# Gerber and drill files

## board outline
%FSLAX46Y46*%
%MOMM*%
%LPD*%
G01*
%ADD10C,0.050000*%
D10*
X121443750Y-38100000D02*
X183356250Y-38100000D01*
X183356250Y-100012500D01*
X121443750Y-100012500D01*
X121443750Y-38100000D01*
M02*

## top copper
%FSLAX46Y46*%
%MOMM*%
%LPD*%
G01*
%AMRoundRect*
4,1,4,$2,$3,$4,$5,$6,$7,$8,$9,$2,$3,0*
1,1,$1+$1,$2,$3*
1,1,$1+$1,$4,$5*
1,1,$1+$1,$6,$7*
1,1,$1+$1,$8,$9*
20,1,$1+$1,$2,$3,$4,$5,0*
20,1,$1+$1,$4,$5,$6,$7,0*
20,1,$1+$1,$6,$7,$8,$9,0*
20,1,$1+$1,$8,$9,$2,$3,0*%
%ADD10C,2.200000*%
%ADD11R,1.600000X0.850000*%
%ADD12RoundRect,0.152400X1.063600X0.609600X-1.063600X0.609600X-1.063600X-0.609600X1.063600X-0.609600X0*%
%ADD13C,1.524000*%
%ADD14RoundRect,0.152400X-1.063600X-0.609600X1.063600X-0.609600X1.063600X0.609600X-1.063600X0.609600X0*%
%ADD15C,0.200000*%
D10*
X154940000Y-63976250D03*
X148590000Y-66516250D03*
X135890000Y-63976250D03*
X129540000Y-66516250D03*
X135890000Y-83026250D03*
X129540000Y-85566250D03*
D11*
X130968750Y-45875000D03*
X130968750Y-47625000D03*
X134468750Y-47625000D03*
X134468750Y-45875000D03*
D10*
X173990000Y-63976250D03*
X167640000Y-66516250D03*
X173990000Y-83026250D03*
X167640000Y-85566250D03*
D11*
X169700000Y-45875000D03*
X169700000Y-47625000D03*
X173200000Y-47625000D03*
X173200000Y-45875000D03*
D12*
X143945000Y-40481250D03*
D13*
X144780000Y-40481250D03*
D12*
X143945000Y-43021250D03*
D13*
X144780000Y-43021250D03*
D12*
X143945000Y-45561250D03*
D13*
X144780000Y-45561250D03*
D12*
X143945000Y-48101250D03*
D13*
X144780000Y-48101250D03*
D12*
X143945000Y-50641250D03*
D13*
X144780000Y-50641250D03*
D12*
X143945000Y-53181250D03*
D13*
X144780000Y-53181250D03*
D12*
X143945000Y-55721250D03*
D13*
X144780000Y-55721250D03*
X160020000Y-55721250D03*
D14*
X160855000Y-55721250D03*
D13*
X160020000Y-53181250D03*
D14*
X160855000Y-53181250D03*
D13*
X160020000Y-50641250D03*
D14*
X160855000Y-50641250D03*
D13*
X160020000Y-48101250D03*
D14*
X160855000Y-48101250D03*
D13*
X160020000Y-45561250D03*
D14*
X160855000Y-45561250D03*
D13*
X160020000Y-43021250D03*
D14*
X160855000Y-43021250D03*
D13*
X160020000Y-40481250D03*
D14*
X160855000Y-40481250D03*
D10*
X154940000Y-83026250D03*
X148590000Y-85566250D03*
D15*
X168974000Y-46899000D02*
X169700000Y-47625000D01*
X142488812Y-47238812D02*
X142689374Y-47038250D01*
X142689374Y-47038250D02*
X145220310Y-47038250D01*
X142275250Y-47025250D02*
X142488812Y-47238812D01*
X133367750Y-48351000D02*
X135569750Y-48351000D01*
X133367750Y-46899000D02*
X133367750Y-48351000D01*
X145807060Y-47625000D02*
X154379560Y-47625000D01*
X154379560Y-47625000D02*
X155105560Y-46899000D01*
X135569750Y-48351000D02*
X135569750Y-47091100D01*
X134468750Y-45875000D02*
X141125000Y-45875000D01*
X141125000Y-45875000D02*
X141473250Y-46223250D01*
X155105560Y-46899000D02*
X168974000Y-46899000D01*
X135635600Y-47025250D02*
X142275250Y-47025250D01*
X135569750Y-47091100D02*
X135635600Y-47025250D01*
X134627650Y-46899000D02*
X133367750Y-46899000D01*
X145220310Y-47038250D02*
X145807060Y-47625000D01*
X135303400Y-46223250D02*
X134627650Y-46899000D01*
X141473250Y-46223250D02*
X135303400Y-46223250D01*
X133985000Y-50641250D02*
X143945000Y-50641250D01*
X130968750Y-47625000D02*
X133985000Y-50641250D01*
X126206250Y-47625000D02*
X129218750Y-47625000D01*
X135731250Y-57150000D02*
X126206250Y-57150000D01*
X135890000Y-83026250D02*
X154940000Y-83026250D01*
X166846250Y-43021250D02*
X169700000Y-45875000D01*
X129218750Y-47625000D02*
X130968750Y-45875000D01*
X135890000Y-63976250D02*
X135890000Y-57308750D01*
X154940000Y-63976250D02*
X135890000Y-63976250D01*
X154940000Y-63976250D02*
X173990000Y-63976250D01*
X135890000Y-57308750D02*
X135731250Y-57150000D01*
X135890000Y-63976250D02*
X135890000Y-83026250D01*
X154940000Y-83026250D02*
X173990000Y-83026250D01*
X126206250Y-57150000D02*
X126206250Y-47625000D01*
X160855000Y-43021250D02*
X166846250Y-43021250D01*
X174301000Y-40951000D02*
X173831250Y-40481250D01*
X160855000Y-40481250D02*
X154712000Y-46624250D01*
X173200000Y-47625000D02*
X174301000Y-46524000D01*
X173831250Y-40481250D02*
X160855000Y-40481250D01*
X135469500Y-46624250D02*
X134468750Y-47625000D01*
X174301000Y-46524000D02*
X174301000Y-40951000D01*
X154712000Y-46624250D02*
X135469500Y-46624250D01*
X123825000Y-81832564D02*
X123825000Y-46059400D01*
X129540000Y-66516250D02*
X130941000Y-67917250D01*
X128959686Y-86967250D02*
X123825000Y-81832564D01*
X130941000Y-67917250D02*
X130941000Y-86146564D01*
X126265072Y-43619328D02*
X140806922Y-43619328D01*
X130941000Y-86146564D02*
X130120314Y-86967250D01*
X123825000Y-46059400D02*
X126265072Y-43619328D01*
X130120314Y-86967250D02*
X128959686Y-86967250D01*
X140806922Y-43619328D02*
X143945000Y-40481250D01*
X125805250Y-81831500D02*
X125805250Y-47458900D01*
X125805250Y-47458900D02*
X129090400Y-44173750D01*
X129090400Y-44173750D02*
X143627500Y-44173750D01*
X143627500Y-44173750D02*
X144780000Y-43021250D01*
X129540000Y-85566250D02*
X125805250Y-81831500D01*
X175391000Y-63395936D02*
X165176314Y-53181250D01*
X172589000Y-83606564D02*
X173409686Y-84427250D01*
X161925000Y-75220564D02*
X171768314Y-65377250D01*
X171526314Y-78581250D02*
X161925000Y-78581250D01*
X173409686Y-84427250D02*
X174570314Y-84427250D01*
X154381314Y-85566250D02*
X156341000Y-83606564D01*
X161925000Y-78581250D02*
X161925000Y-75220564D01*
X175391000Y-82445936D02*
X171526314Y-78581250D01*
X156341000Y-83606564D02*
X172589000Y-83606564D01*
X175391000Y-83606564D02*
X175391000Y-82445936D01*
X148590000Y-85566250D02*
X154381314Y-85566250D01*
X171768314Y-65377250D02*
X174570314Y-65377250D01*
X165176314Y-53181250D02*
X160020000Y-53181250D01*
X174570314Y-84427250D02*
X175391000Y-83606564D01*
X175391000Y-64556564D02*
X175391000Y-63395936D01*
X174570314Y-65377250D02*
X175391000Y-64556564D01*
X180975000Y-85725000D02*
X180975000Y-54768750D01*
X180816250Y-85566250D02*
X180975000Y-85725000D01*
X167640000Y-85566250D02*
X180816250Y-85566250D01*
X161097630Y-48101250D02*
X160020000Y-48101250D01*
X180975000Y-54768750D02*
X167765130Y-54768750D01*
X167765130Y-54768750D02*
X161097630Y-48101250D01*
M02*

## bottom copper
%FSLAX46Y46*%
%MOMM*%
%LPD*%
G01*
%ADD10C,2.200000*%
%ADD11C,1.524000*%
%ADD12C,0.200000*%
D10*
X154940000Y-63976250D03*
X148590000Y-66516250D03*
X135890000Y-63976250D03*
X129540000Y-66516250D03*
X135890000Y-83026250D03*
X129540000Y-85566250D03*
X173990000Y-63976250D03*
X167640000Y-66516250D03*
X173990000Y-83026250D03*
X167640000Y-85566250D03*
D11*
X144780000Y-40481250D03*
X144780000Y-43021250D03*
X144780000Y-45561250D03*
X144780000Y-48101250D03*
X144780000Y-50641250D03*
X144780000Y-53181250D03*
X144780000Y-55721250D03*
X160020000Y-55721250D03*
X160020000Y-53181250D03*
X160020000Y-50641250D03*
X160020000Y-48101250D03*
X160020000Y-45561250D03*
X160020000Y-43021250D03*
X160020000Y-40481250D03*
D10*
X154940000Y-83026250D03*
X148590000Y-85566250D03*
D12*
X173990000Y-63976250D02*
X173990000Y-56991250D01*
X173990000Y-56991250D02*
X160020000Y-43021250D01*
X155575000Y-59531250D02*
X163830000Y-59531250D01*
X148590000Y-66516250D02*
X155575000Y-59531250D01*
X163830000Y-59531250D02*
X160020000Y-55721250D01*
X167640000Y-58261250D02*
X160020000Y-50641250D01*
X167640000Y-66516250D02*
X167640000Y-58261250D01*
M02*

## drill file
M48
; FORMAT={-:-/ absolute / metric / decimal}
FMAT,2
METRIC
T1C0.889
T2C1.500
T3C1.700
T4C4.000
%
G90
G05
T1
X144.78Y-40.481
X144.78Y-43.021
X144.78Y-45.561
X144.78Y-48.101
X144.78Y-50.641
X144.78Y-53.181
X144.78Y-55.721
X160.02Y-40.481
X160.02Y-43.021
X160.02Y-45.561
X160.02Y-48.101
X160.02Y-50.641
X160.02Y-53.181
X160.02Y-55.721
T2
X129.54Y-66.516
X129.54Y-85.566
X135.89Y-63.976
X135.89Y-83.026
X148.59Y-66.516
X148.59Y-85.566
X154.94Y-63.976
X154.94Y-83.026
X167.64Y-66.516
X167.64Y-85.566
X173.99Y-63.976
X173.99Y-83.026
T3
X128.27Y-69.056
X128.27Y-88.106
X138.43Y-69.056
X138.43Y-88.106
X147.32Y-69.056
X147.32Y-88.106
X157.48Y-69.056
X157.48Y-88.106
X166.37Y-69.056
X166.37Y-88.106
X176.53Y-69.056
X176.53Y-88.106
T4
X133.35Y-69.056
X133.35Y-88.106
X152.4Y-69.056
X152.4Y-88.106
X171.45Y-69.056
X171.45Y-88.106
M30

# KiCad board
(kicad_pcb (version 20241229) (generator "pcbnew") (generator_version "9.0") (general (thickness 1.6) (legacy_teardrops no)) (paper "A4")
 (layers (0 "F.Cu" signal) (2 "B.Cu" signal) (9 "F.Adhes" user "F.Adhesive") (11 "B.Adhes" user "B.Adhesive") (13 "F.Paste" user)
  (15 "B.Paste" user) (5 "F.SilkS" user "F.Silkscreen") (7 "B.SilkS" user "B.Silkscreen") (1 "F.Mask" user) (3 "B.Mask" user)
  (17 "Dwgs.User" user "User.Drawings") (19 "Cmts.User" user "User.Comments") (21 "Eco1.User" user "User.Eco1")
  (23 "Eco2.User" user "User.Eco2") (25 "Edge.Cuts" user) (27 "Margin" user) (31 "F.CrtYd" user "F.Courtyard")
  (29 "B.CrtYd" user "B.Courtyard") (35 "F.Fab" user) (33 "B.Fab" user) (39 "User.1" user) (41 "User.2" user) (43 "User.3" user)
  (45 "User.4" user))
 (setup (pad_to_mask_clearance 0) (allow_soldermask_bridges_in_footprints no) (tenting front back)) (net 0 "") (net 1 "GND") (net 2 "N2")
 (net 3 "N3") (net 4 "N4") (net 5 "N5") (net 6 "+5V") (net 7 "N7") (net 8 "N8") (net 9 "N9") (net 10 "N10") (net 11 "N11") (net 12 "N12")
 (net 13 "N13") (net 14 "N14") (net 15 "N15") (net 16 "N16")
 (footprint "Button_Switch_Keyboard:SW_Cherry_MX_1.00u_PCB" (layer "F.Cu") (at 154.94 63.97625)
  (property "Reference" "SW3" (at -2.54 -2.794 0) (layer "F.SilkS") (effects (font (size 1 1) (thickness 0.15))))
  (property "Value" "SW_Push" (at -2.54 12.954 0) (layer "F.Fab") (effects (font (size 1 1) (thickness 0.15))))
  (pad "" np_thru_hole circle (at -7.62 5.08) (size 1.7 1.7) (drill 1.7) (layers "*.Cu" "*.Mask"))
  (pad "" np_thru_hole circle (at -2.54 5.08) (size 4 4) (drill 4) (layers "*.Cu" "*.Mask"))
  (pad "" np_thru_hole circle (at 2.54 5.08) (size 1.7 1.7) (drill 1.7) (layers "*.Cu" "*.Mask"))
  (pad "1" thru_hole circle (at 0 0) (size 2.2 2.2) (drill 1.5) (layers "*.Cu" "*.Mask") (remove_unused_layers no) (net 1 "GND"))
  (pad "2" thru_hole circle (at -6.35 2.54) (size 2.2 2.2) (drill 1.5) (layers "*.Cu" "*.Mask") (remove_unused_layers no) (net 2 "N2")))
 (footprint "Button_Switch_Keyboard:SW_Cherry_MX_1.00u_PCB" (layer "F.Cu") (at 135.89 63.97625)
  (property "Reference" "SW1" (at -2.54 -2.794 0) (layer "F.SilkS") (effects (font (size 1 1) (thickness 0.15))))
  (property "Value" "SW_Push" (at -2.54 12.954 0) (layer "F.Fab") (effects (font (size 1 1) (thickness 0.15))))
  (pad "" np_thru_hole circle (at -7.62 5.08) (size 1.7 1.7) (drill 1.7) (layers "*.Cu" "*.Mask"))
  (pad "" np_thru_hole circle (at -2.54 5.08) (size 4 4) (drill 4) (layers "*.Cu" "*.Mask"))
  (pad "" np_thru_hole circle (at 2.54 5.08) (size 1.7 1.7) (drill 1.7) (layers "*.Cu" "*.Mask"))
  (pad "1" thru_hole circle (at 0 0) (size 2.2 2.2) (drill 1.5) (layers "*.Cu" "*.Mask") (remove_unused_layers no) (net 1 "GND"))
  (pad "2" thru_hole circle (at -6.35 2.54) (size 2.2 2.2) (drill 1.5) (layers "*.Cu" "*.Mask") (remove_unused_layers no) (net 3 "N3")))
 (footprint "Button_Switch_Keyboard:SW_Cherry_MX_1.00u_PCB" (layer "F.Cu") (at 135.89 83.02625)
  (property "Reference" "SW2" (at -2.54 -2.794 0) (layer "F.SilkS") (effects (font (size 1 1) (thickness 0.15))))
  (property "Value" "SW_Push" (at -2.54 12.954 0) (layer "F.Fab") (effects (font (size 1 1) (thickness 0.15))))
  (pad "" np_thru_hole circle (at -7.62 5.08) (size 1.7 1.7) (drill 1.7) (layers "*.Cu" "*.Mask"))
  (pad "" np_thru_hole circle (at -2.54 5.08) (size 4 4) (drill 4) (layers "*.Cu" "*.Mask"))
  (pad "" np_thru_hole circle (at 2.54 5.08) (size 1.7 1.7) (drill 1.7) (layers "*.Cu" "*.Mask"))
  (pad "1" thru_hole circle (at 0 0) (size 2.2 2.2) (drill 1.5) (layers "*.Cu" "*.Mask") (remove_unused_layers no) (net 1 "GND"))
  (pad "2" thru_hole circle (at -6.35 2.54) (size 2.2 2.2) (drill 1.5) (layers "*.Cu" "*.Mask") (remove_unused_layers no) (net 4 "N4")))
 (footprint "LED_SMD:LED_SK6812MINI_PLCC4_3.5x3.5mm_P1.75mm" (layer "F.Cu") (at 132.71875 46.75)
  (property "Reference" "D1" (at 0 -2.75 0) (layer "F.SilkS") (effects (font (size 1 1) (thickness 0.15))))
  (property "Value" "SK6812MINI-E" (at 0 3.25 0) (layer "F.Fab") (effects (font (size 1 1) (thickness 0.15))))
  (pad "1" smd rect (at -1.75 -0.875) (size 1.6 0.85) (layers "F.Cu" "F.Mask" "F.Paste") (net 1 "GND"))
  (pad "2" smd rect (at -1.75 0.875) (size 1.6 0.85) (layers "F.Cu" "F.Mask" "F.Paste") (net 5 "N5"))
  (pad "3" smd rect (at 1.75 0.875) (size 1.6 0.85) (layers "F.Cu" "F.Mask" "F.Paste") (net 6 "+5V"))
  (pad "4" smd rect (at 1.75 -0.875) (size 1.6 0.85) (layers "F.Cu" "F.Mask" "F.Paste") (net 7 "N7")))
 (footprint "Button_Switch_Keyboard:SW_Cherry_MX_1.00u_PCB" (layer "F.Cu") (at 173.99 63.97625)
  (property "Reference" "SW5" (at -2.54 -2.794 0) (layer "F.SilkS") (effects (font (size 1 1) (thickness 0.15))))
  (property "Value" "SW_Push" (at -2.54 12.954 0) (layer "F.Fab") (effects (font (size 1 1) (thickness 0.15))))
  (pad "" np_thru_hole circle (at -7.62 5.08) (size 1.7 1.7) (drill 1.7) (layers "*.Cu" "*.Mask"))
  (pad "" np_thru_hole circle (at -2.54 5.08) (size 4 4) (drill 4) (layers "*.Cu" "*.Mask"))
  (pad "" np_thru_hole circle (at 2.54 5.08) (size 1.7 1.7) (drill 1.7) (layers "*.Cu" "*.Mask"))
  (pad "1" thru_hole circle (at 0 0) (size 2.2 2.2) (drill 1.5) (layers "*.Cu" "*.Mask") (remove_unused_layers no) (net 1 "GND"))
  (pad "2" thru_hole circle (at -6.35 2.54) (size 2.2 2.2) (drill 1.5) (layers "*.Cu" "*.Mask") (remove_unused_layers no) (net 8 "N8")))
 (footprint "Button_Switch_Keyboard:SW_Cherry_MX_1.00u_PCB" (layer "F.Cu") (at 173.99 83.02625)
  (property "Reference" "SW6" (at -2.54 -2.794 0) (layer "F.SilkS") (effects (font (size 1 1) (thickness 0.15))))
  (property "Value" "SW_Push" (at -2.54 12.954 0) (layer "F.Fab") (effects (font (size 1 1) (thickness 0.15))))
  (pad "" np_thru_hole circle (at -7.62 5.08) (size 1.7 1.7) (drill 1.7) (layers "*.Cu" "*.Mask"))
  (pad "" np_thru_hole circle (at -2.54 5.08) (size 4 4) (drill 4) (layers "*.Cu" "*.Mask"))
  (pad "" np_thru_hole circle (at 2.54 5.08) (size 1.7 1.7) (drill 1.7) (layers "*.Cu" "*.Mask"))
  (pad "1" thru_hole circle (at 0 0) (size 2.2 2.2) (drill 1.5) (layers "*.Cu" "*.Mask") (remove_unused_layers no) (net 1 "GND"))
  (pad "2" thru_hole circle (at -6.35 2.54) (size 2.2 2.2) (drill 1.5) (layers "*.Cu" "*.Mask") (remove_unused_layers no) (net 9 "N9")))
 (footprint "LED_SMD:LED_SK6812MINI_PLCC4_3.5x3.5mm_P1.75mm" (layer "F.Cu") (at 171.45 46.75)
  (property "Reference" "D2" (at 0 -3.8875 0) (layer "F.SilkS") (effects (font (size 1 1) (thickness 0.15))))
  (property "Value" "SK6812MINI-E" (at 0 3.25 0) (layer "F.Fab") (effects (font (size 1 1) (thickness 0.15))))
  (pad "1" smd rect (at -1.75 -0.875) (size 1.6 0.85) (layers "F.Cu" "F.Mask" "F.Paste") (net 1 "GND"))
  (pad "2" smd rect (at -1.75 0.875) (size 1.6 0.85) (layers "F.Cu" "F.Mask" "F.Paste") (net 7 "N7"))
  (pad "3" smd rect (at 1.75 0.875) (size 1.6 0.85) (layers "F.Cu" "F.Mask" "F.Paste") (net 6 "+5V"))
  (pad "4" smd rect (at 1.75 -0.875) (size 1.6 0.85) (layers "F.Cu" "F.Mask" "F.Paste") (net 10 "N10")))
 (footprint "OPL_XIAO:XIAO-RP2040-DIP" (layer "F.Cu") (at 152.4 48.10125)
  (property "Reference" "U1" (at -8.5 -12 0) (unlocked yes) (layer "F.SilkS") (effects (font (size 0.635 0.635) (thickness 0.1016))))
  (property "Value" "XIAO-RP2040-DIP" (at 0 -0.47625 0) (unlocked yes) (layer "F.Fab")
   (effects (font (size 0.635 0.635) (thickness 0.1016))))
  (pad "1" smd roundrect (at -8.455 -7.62 180) (size 2.432 1.524) (layers "F.Cu" "F.Mask") (roundrect_rratio 0.1) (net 3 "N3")
   (thermal_bridge_angle 45))
  (pad "1" thru_hole circle (at -7.62 -7.62 180) (size 1.524 1.524) (drill 0.889) (layers "*.Cu" "*.Mask") (remove_unused_layers no)
   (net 3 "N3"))
  (pad "2" smd roundrect (at -8.455 -5.08 180) (size 2.432 1.524) (layers "F.Cu" "F.Mask") (roundrect_rratio 0.1) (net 4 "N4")
   (thermal_bridge_angle 45))
  (pad "2" thru_hole circle (at -7.62 -5.08 180) (size 1.524 1.524) (drill 0.889) (layers "*.Cu" "*.Mask") (remove_unused_layers no)
   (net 4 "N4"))
  (pad "3" smd roundrect (at -8.455 -2.54 180) (size 2.432 1.524) (layers "F.Cu" "F.Mask") (roundrect_rratio 0.1) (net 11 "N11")
   (thermal_bridge_angle 45))
  (pad "3" thru_hole circle (at -7.62 -2.54 180) (size 1.524 1.524) (drill 0.889) (layers "*.Cu" "*.Mask") (remove_unused_layers no)
   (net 11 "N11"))
  (pad "4" smd roundrect (at -8.455 0 180) (size 2.432 1.524) (layers "F.Cu" "F.Mask") (roundrect_rratio 0.1) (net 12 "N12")
   (thermal_bridge_angle 45))
  (pad "4" thru_hole circle (at -7.62 0 180) (size 1.524 1.524) (drill 0.889) (layers "*.Cu" "*.Mask") (remove_unused_layers no)
   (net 12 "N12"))
  (pad "5" smd roundrect (at -8.455 2.54 180) (size 2.432 1.524) (layers "F.Cu" "F.Mask") (roundrect_rratio 0.1) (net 5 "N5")
   (thermal_bridge_angle 45))
  (pad "5" thru_hole circle (at -7.62 2.54 180) (size 1.524 1.524) (drill 0.889) (layers "*.Cu" "*.Mask") (remove_unused_layers no)
   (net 5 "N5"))
  (pad "6" smd roundrect (at -8.455 5.08 180) (size 2.432 1.524) (layers "F.Cu" "F.Mask") (roundrect_rratio 0.1) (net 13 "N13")
   (thermal_bridge_angle 45))
  (pad "6" thru_hole circle (at -7.62 5.08 180) (size 1.524 1.524) (drill 0.889) (layers "*.Cu" "*.Mask") (remove_unused_layers no)
   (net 13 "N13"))
  (pad "7" smd roundrect (at -8.455 7.62 180) (size 2.432 1.524) (layers "F.Cu" "F.Mask") (roundrect_rratio 0.1) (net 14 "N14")
   (thermal_bridge_angle 45))
  (pad "7" thru_hole circle (at -7.62 7.62 180) (size 1.524 1.524) (drill 0.889) (layers "*.Cu" "*.Mask") (remove_unused_layers no)
   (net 14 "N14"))
  (pad "8" thru_hole circle (at 7.62 7.62) (size 1.524 1.524) (drill 0.889) (layers "*.Cu" "*.Mask") (remove_unused_layers no) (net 2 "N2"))
  (pad "8" smd roundrect (at 8.455 7.62) (size 2.432 1.524) (layers "F.Cu" "F.Mask") (roundrect_rratio 0.1) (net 2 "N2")
   (thermal_bridge_angle 45))
  (pad "9" thru_hole circle (at 7.62 5.08) (size 1.524 1.524) (drill 0.889) (layers "*.Cu" "*.Mask") (remove_unused_layers no)
   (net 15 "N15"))
  (pad "9" smd roundrect (at 8.455 5.08) (size 2.432 1.524) (layers "F.Cu" "F.Mask") (roundrect_rratio 0.1) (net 15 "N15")
   (thermal_bridge_angle 45))
  (pad "10" thru_hole circle (at 7.62 2.54) (size 1.524 1.524) (drill 0.889) (layers "*.Cu" "*.Mask") (remove_unused_layers no) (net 8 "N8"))
  (pad "10" smd roundrect (at 8.455 2.54) (size 2.432 1.524) (layers "F.Cu" "F.Mask") (roundrect_rratio 0.1) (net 8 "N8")
   (thermal_bridge_angle 45))
  (pad "11" thru_hole circle (at 7.62 0) (size 1.524 1.524) (drill 0.889) (layers "*.Cu" "*.Mask") (remove_unused_layers no) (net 9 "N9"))
  (pad "11" smd roundrect (at 8.455 0) (size 2.432 1.524) (layers "F.Cu" "F.Mask") (roundrect_rratio 0.1) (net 9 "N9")
   (thermal_bridge_angle 45))
  (pad "12" thru_hole circle (at 7.62 -2.54) (size 1.524 1.524) (drill 0.889) (layers "*.Cu" "*.Mask") (remove_unused_layers no)
   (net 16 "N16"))
  (pad "12" smd roundrect (at 8.455 -2.54) (size 2.432 1.524) (layers "F.Cu" "F.Mask") (roundrect_rratio 0.1) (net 16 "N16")
   (thermal_bridge_angle 45))
  (pad "13" thru_hole circle (at 7.62 -5.08) (size 1.524 1.524) (drill 0.889) (layers "*.Cu" "*.Mask") (remove_unused_layers no)
   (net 1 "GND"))
  (pad "13" smd roundrect (at 8.455 -5.08) (size 2.432 1.524) (layers "F.Cu" "F.Mask") (roundrect_rratio 0.1) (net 1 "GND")
   (thermal_bridge_angle 45))
  (pad "14" thru_hole circle (at 7.62 -7.62) (size 1.524 1.524) (drill 0.889) (layers "*.Cu" "*.Mask") (remove_unused_layers no)
   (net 6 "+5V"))
  (pad "14" smd roundrect (at 8.455 -7.62) (size 2.432 1.524) (layers "F.Cu" "F.Mask") (roundrect_rratio 0.1) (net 6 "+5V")
   (thermal_bridge_angle 45)))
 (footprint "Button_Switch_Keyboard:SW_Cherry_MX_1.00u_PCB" (layer "F.Cu") (at 154.94 83.02625)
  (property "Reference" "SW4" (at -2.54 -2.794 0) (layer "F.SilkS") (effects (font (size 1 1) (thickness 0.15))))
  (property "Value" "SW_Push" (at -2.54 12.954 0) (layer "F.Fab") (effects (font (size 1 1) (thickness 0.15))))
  (pad "" np_thru_hole circle (at -7.62 5.08) (size 1.7 1.7) (drill 1.7) (layers "*.Cu" "*.Mask"))
  (pad "" np_thru_hole circle (at -2.54 5.08) (size 4 4) (drill 4) (layers "*.Cu" "*.Mask"))
  (pad "" np_thru_hole circle (at 2.54 5.08) (size 1.7 1.7) (drill 1.7) (layers "*.Cu" "*.Mask"))
  (pad "1" thru_hole circle (at 0 0) (size 2.2 2.2) (drill 1.5) (layers "*.Cu" "*.Mask") (remove_unused_layers no) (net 1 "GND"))
  (pad "2" thru_hole circle (at -6.35 2.54) (size 2.2 2.2) (drill 1.5) (layers "*.Cu" "*.Mask") (remove_unused_layers no) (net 15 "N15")))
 (gr_rect (start 121.44375 38.1) (end 183.35625 100.0125) (stroke (width 0.05) (type default)) (fill no) (layer "Edge.Cuts"))
 (segment (start 168.974 46.899) (end 169.7 47.625) (width 0.2) (layer "F.Cu") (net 7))
 (segment (start 142.488812 47.238812) (end 142.689374 47.03825) (width 0.2) (layer "F.Cu") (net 7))
 (segment (start 142.689374 47.03825) (end 145.22031 47.03825) (width 0.2) (layer "F.Cu") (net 7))
 (segment (start 142.27525 47.02525) (end 142.488812 47.238812) (width 0.2) (layer "F.Cu") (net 7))
 (segment (start 133.36775 48.351) (end 135.56975 48.351) (width 0.2) (layer "F.Cu") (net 7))
 (segment (start 133.36775 46.899) (end 133.36775 48.351) (width 0.2) (layer "F.Cu") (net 7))
 (segment (start 145.80706 47.625) (end 154.37956 47.625) (width 0.2) (layer "F.Cu") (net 7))
 (segment (start 154.37956 47.625) (end 155.10556 46.899) (width 0.2) (layer "F.Cu") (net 7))
 (segment (start 135.56975 48.351) (end 135.56975 47.0911) (width 0.2) (layer "F.Cu") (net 7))
 (segment (start 134.46875 45.875) (end 141.125 45.875) (width 0.2) (layer "F.Cu") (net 7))
 (segment (start 141.125 45.875) (end 141.47325 46.22325) (width 0.2) (layer "F.Cu") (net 7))
 (segment (start 155.10556 46.899) (end 168.974 46.899) (width 0.2) (layer "F.Cu") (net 7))
 (segment (start 135.6356 47.02525) (end 142.27525 47.02525) (width 0.2) (layer "F.Cu") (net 7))
 (segment (start 135.56975 47.0911) (end 135.6356 47.02525) (width 0.2) (layer "F.Cu") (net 7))
 (segment (start 134.62765 46.899) (end 133.36775 46.899) (width 0.2) (layer "F.Cu") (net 7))
 (segment (start 145.22031 47.03825) (end 145.80706 47.625) (width 0.2) (layer "F.Cu") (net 7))
 (segment (start 135.3034 46.22325) (end 134.62765 46.899) (width 0.2) (layer "F.Cu") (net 7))
 (segment (start 141.47325 46.22325) (end 135.3034 46.22325) (width 0.2) (layer "F.Cu") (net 7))
 (segment (start 133.985 50.64125) (end 143.945 50.64125) (width 0.2) (layer "F.Cu") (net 5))
 (segment (start 130.96875 47.625) (end 133.985 50.64125) (width 0.2) (layer "F.Cu") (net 5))
 (segment (start 126.20625 47.625) (end 129.21875 47.625) (width 0.2) (layer "F.Cu") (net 1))
 (segment (start 135.73125 57.15) (end 126.20625 57.15) (width 0.2) (layer "F.Cu") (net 1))
 (segment (start 135.89 83.02625) (end 154.94 83.02625) (width 0.2) (layer "F.Cu") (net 1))
 (segment (start 166.84625 43.02125) (end 169.7 45.875) (width 0.2) (layer "F.Cu") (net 1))
 (segment (start 129.21875 47.625) (end 130.96875 45.875) (width 0.2) (layer "F.Cu") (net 1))
 (segment (start 135.89 63.97625) (end 135.89 57.30875) (width 0.2) (layer "F.Cu") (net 1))
 (segment (start 154.94 63.97625) (end 135.89 63.97625) (width 0.2) (layer "F.Cu") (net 1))
 (segment (start 154.94 63.97625) (end 173.99 63.97625) (width 0.2) (layer "F.Cu") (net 1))
 (segment (start 135.89 57.30875) (end 135.73125 57.15) (width 0.2) (layer "F.Cu") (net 1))
 (segment (start 135.89 63.97625) (end 135.89 83.02625) (width 0.2) (layer "F.Cu") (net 1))
 (segment (start 154.94 83.02625) (end 173.99 83.02625) (width 0.2) (layer "F.Cu") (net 1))
 (segment (start 126.20625 57.15) (end 126.20625 47.625) (width 0.2) (layer "F.Cu") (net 1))
 (segment (start 160.855 43.02125) (end 166.84625 43.02125) (width 0.2) (layer "F.Cu") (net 1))
 (segment (start 173.99 63.97625) (end 173.99 56.99125) (width 0.2) (layer "B.Cu") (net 1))
 (segment (start 173.99 56.99125) (end 160.02 43.02125) (width 0.2) (layer "B.Cu") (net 1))
 (segment (start 174.301 40.951) (end 173.83125 40.48125) (width 0.2) (layer "F.Cu") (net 6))
 (segment (start 160.855 40.48125) (end 154.712 46.62425) (width 0.2) (layer "F.Cu") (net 6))
 (segment (start 173.2 47.625) (end 174.301 46.524) (width 0.2) (layer "F.Cu") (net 6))
 (segment (start 173.83125 40.48125) (end 160.855 40.48125) (width 0.2) (layer "F.Cu") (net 6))
 (segment (start 135.4695 46.62425) (end 134.46875 47.625) (width 0.2) (layer "F.Cu") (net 6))
 (segment (start 174.301 46.524) (end 174.301 40.951) (width 0.2) (layer "F.Cu") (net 6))
 (segment (start 154.712 46.62425) (end 135.4695 46.62425) (width 0.2) (layer "F.Cu") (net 6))
 (segment (start 123.825 81.832564) (end 123.825 46.0594) (width 0.2) (layer "F.Cu") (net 3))
 (segment (start 129.54 66.51625) (end 130.941 67.91725) (width 0.2) (layer "F.Cu") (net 3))
 (segment (start 128.959686 86.96725) (end 123.825 81.832564) (width 0.2) (layer "F.Cu") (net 3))
 (segment (start 130.941 67.91725) (end 130.941 86.146564) (width 0.2) (layer "F.Cu") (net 3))
 (segment (start 126.265072 43.619328) (end 140.806922 43.619328) (width 0.2) (layer "F.Cu") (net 3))
 (segment (start 130.941 86.146564) (end 130.120314 86.96725) (width 0.2) (layer "F.Cu") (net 3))
 (segment (start 123.825 46.0594) (end 126.265072 43.619328) (width 0.2) (layer "F.Cu") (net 3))
 (segment (start 130.120314 86.96725) (end 128.959686 86.96725) (width 0.2) (layer "F.Cu") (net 3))
 (segment (start 140.806922 43.619328) (end 143.945 40.48125) (width 0.2) (layer "F.Cu") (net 3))
 (segment (start 125.80525 81.8315) (end 125.80525 47.4589) (width 0.2) (layer "F.Cu") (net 4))
 (segment (start 125.80525 47.4589) (end 129.0904 44.17375) (width 0.2) (layer "F.Cu") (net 4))
 (segment (start 129.0904 44.17375) (end 143.6275 44.17375) (width 0.2) (layer "F.Cu") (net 4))
 (segment (start 143.6275 44.17375) (end 144.78 43.02125) (width 0.2) (layer "F.Cu") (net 4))
 (segment (start 129.54 85.56625) (end 125.80525 81.8315) (width 0.2) (layer "F.Cu") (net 4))
 (segment (start 155.575 59.53125) (end 163.83 59.53125) (width 0.2) (layer "B.Cu") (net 2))
 (segment (start 148.59 66.51625) (end 155.575 59.53125) (width 0.2) (layer "B.Cu") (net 2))
 (segment (start 163.83 59.53125) (end 160.02 55.72125) (width 0.2) (layer "B.Cu") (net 2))
 (segment (start 175.391 63.395936) (end 165.176314 53.18125) (width 0.2) (layer "F.Cu") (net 15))
 (segment (start 172.589 83.606564) (end 173.409686 84.42725) (width 0.2) (layer "F.Cu") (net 15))
 (segment (start 161.925 75.220564) (end 171.768314 65.37725) (width 0.2) (layer "F.Cu") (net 15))
 (segment (start 171.526314 78.58125) (end 161.925 78.58125) (width 0.2) (layer "F.Cu") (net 15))
 (segment (start 173.409686 84.42725) (end 174.570314 84.42725) (width 0.2) (layer "F.Cu") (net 15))
 (segment (start 154.381314 85.56625) (end 156.341 83.606564) (width 0.2) (layer "F.Cu") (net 15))
 (segment (start 161.925 78.58125) (end 161.925 75.220564) (width 0.2) (layer "F.Cu") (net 15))
 (segment (start 175.391 82.445936) (end 171.526314 78.58125) (width 0.2) (layer "F.Cu") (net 15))
 (segment (start 156.341 83.606564) (end 172.589 83.606564) (width 0.2) (layer "F.Cu") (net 15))
 (segment (start 175.391 83.606564) (end 175.391 82.445936) (width 0.2) (layer "F.Cu") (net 15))
 (segment (start 148.59 85.56625) (end 154.381314 85.56625) (width 0.2) (layer "F.Cu") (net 15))
 (segment (start 171.768314 65.37725) (end 174.570314 65.37725) (width 0.2) (layer "F.Cu") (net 15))
 (segment (start 165.176314 53.18125) (end 160.02 53.18125) (width 0.2) (layer "F.Cu") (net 15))
 (segment (start 174.570314 84.42725) (end 175.391 83.606564) (width 0.2) (layer "F.Cu") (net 15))
 (segment (start 175.391 64.556564) (end 175.391 63.395936) (width 0.2) (layer "F.Cu") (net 15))
 (segment (start 174.570314 65.37725) (end 175.391 64.556564) (width 0.2) (layer "F.Cu") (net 15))
 (segment (start 167.64 58.26125) (end 160.02 50.64125) (width 0.2) (layer "B.Cu") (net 8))
 (segment (start 167.64 66.51625) (end 167.64 58.26125) (width 0.2) (layer "B.Cu") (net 8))
 (segment (start 180.975 85.725) (end 180.975 54.76875) (width 0.2) (layer "F.Cu") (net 9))
 (segment (start 180.81625 85.56625) (end 180.975 85.725) (width 0.2) (layer "F.Cu") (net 9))
 (segment (start 167.64 85.56625) (end 180.81625 85.56625) (width 0.2) (layer "F.Cu") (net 9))
 (segment (start 161.09763 48.10125) (end 160.02 48.10125) (width 0.2) (layer "F.Cu") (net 9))
 (segment (start 180.975 54.76875) (end 167.76513 54.76875) (width 0.2) (layer "F.Cu") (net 9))
 (segment (start 167.76513 54.76875) (end 161.09763 48.10125) (width 0.2) (layer "F.Cu") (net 9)))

